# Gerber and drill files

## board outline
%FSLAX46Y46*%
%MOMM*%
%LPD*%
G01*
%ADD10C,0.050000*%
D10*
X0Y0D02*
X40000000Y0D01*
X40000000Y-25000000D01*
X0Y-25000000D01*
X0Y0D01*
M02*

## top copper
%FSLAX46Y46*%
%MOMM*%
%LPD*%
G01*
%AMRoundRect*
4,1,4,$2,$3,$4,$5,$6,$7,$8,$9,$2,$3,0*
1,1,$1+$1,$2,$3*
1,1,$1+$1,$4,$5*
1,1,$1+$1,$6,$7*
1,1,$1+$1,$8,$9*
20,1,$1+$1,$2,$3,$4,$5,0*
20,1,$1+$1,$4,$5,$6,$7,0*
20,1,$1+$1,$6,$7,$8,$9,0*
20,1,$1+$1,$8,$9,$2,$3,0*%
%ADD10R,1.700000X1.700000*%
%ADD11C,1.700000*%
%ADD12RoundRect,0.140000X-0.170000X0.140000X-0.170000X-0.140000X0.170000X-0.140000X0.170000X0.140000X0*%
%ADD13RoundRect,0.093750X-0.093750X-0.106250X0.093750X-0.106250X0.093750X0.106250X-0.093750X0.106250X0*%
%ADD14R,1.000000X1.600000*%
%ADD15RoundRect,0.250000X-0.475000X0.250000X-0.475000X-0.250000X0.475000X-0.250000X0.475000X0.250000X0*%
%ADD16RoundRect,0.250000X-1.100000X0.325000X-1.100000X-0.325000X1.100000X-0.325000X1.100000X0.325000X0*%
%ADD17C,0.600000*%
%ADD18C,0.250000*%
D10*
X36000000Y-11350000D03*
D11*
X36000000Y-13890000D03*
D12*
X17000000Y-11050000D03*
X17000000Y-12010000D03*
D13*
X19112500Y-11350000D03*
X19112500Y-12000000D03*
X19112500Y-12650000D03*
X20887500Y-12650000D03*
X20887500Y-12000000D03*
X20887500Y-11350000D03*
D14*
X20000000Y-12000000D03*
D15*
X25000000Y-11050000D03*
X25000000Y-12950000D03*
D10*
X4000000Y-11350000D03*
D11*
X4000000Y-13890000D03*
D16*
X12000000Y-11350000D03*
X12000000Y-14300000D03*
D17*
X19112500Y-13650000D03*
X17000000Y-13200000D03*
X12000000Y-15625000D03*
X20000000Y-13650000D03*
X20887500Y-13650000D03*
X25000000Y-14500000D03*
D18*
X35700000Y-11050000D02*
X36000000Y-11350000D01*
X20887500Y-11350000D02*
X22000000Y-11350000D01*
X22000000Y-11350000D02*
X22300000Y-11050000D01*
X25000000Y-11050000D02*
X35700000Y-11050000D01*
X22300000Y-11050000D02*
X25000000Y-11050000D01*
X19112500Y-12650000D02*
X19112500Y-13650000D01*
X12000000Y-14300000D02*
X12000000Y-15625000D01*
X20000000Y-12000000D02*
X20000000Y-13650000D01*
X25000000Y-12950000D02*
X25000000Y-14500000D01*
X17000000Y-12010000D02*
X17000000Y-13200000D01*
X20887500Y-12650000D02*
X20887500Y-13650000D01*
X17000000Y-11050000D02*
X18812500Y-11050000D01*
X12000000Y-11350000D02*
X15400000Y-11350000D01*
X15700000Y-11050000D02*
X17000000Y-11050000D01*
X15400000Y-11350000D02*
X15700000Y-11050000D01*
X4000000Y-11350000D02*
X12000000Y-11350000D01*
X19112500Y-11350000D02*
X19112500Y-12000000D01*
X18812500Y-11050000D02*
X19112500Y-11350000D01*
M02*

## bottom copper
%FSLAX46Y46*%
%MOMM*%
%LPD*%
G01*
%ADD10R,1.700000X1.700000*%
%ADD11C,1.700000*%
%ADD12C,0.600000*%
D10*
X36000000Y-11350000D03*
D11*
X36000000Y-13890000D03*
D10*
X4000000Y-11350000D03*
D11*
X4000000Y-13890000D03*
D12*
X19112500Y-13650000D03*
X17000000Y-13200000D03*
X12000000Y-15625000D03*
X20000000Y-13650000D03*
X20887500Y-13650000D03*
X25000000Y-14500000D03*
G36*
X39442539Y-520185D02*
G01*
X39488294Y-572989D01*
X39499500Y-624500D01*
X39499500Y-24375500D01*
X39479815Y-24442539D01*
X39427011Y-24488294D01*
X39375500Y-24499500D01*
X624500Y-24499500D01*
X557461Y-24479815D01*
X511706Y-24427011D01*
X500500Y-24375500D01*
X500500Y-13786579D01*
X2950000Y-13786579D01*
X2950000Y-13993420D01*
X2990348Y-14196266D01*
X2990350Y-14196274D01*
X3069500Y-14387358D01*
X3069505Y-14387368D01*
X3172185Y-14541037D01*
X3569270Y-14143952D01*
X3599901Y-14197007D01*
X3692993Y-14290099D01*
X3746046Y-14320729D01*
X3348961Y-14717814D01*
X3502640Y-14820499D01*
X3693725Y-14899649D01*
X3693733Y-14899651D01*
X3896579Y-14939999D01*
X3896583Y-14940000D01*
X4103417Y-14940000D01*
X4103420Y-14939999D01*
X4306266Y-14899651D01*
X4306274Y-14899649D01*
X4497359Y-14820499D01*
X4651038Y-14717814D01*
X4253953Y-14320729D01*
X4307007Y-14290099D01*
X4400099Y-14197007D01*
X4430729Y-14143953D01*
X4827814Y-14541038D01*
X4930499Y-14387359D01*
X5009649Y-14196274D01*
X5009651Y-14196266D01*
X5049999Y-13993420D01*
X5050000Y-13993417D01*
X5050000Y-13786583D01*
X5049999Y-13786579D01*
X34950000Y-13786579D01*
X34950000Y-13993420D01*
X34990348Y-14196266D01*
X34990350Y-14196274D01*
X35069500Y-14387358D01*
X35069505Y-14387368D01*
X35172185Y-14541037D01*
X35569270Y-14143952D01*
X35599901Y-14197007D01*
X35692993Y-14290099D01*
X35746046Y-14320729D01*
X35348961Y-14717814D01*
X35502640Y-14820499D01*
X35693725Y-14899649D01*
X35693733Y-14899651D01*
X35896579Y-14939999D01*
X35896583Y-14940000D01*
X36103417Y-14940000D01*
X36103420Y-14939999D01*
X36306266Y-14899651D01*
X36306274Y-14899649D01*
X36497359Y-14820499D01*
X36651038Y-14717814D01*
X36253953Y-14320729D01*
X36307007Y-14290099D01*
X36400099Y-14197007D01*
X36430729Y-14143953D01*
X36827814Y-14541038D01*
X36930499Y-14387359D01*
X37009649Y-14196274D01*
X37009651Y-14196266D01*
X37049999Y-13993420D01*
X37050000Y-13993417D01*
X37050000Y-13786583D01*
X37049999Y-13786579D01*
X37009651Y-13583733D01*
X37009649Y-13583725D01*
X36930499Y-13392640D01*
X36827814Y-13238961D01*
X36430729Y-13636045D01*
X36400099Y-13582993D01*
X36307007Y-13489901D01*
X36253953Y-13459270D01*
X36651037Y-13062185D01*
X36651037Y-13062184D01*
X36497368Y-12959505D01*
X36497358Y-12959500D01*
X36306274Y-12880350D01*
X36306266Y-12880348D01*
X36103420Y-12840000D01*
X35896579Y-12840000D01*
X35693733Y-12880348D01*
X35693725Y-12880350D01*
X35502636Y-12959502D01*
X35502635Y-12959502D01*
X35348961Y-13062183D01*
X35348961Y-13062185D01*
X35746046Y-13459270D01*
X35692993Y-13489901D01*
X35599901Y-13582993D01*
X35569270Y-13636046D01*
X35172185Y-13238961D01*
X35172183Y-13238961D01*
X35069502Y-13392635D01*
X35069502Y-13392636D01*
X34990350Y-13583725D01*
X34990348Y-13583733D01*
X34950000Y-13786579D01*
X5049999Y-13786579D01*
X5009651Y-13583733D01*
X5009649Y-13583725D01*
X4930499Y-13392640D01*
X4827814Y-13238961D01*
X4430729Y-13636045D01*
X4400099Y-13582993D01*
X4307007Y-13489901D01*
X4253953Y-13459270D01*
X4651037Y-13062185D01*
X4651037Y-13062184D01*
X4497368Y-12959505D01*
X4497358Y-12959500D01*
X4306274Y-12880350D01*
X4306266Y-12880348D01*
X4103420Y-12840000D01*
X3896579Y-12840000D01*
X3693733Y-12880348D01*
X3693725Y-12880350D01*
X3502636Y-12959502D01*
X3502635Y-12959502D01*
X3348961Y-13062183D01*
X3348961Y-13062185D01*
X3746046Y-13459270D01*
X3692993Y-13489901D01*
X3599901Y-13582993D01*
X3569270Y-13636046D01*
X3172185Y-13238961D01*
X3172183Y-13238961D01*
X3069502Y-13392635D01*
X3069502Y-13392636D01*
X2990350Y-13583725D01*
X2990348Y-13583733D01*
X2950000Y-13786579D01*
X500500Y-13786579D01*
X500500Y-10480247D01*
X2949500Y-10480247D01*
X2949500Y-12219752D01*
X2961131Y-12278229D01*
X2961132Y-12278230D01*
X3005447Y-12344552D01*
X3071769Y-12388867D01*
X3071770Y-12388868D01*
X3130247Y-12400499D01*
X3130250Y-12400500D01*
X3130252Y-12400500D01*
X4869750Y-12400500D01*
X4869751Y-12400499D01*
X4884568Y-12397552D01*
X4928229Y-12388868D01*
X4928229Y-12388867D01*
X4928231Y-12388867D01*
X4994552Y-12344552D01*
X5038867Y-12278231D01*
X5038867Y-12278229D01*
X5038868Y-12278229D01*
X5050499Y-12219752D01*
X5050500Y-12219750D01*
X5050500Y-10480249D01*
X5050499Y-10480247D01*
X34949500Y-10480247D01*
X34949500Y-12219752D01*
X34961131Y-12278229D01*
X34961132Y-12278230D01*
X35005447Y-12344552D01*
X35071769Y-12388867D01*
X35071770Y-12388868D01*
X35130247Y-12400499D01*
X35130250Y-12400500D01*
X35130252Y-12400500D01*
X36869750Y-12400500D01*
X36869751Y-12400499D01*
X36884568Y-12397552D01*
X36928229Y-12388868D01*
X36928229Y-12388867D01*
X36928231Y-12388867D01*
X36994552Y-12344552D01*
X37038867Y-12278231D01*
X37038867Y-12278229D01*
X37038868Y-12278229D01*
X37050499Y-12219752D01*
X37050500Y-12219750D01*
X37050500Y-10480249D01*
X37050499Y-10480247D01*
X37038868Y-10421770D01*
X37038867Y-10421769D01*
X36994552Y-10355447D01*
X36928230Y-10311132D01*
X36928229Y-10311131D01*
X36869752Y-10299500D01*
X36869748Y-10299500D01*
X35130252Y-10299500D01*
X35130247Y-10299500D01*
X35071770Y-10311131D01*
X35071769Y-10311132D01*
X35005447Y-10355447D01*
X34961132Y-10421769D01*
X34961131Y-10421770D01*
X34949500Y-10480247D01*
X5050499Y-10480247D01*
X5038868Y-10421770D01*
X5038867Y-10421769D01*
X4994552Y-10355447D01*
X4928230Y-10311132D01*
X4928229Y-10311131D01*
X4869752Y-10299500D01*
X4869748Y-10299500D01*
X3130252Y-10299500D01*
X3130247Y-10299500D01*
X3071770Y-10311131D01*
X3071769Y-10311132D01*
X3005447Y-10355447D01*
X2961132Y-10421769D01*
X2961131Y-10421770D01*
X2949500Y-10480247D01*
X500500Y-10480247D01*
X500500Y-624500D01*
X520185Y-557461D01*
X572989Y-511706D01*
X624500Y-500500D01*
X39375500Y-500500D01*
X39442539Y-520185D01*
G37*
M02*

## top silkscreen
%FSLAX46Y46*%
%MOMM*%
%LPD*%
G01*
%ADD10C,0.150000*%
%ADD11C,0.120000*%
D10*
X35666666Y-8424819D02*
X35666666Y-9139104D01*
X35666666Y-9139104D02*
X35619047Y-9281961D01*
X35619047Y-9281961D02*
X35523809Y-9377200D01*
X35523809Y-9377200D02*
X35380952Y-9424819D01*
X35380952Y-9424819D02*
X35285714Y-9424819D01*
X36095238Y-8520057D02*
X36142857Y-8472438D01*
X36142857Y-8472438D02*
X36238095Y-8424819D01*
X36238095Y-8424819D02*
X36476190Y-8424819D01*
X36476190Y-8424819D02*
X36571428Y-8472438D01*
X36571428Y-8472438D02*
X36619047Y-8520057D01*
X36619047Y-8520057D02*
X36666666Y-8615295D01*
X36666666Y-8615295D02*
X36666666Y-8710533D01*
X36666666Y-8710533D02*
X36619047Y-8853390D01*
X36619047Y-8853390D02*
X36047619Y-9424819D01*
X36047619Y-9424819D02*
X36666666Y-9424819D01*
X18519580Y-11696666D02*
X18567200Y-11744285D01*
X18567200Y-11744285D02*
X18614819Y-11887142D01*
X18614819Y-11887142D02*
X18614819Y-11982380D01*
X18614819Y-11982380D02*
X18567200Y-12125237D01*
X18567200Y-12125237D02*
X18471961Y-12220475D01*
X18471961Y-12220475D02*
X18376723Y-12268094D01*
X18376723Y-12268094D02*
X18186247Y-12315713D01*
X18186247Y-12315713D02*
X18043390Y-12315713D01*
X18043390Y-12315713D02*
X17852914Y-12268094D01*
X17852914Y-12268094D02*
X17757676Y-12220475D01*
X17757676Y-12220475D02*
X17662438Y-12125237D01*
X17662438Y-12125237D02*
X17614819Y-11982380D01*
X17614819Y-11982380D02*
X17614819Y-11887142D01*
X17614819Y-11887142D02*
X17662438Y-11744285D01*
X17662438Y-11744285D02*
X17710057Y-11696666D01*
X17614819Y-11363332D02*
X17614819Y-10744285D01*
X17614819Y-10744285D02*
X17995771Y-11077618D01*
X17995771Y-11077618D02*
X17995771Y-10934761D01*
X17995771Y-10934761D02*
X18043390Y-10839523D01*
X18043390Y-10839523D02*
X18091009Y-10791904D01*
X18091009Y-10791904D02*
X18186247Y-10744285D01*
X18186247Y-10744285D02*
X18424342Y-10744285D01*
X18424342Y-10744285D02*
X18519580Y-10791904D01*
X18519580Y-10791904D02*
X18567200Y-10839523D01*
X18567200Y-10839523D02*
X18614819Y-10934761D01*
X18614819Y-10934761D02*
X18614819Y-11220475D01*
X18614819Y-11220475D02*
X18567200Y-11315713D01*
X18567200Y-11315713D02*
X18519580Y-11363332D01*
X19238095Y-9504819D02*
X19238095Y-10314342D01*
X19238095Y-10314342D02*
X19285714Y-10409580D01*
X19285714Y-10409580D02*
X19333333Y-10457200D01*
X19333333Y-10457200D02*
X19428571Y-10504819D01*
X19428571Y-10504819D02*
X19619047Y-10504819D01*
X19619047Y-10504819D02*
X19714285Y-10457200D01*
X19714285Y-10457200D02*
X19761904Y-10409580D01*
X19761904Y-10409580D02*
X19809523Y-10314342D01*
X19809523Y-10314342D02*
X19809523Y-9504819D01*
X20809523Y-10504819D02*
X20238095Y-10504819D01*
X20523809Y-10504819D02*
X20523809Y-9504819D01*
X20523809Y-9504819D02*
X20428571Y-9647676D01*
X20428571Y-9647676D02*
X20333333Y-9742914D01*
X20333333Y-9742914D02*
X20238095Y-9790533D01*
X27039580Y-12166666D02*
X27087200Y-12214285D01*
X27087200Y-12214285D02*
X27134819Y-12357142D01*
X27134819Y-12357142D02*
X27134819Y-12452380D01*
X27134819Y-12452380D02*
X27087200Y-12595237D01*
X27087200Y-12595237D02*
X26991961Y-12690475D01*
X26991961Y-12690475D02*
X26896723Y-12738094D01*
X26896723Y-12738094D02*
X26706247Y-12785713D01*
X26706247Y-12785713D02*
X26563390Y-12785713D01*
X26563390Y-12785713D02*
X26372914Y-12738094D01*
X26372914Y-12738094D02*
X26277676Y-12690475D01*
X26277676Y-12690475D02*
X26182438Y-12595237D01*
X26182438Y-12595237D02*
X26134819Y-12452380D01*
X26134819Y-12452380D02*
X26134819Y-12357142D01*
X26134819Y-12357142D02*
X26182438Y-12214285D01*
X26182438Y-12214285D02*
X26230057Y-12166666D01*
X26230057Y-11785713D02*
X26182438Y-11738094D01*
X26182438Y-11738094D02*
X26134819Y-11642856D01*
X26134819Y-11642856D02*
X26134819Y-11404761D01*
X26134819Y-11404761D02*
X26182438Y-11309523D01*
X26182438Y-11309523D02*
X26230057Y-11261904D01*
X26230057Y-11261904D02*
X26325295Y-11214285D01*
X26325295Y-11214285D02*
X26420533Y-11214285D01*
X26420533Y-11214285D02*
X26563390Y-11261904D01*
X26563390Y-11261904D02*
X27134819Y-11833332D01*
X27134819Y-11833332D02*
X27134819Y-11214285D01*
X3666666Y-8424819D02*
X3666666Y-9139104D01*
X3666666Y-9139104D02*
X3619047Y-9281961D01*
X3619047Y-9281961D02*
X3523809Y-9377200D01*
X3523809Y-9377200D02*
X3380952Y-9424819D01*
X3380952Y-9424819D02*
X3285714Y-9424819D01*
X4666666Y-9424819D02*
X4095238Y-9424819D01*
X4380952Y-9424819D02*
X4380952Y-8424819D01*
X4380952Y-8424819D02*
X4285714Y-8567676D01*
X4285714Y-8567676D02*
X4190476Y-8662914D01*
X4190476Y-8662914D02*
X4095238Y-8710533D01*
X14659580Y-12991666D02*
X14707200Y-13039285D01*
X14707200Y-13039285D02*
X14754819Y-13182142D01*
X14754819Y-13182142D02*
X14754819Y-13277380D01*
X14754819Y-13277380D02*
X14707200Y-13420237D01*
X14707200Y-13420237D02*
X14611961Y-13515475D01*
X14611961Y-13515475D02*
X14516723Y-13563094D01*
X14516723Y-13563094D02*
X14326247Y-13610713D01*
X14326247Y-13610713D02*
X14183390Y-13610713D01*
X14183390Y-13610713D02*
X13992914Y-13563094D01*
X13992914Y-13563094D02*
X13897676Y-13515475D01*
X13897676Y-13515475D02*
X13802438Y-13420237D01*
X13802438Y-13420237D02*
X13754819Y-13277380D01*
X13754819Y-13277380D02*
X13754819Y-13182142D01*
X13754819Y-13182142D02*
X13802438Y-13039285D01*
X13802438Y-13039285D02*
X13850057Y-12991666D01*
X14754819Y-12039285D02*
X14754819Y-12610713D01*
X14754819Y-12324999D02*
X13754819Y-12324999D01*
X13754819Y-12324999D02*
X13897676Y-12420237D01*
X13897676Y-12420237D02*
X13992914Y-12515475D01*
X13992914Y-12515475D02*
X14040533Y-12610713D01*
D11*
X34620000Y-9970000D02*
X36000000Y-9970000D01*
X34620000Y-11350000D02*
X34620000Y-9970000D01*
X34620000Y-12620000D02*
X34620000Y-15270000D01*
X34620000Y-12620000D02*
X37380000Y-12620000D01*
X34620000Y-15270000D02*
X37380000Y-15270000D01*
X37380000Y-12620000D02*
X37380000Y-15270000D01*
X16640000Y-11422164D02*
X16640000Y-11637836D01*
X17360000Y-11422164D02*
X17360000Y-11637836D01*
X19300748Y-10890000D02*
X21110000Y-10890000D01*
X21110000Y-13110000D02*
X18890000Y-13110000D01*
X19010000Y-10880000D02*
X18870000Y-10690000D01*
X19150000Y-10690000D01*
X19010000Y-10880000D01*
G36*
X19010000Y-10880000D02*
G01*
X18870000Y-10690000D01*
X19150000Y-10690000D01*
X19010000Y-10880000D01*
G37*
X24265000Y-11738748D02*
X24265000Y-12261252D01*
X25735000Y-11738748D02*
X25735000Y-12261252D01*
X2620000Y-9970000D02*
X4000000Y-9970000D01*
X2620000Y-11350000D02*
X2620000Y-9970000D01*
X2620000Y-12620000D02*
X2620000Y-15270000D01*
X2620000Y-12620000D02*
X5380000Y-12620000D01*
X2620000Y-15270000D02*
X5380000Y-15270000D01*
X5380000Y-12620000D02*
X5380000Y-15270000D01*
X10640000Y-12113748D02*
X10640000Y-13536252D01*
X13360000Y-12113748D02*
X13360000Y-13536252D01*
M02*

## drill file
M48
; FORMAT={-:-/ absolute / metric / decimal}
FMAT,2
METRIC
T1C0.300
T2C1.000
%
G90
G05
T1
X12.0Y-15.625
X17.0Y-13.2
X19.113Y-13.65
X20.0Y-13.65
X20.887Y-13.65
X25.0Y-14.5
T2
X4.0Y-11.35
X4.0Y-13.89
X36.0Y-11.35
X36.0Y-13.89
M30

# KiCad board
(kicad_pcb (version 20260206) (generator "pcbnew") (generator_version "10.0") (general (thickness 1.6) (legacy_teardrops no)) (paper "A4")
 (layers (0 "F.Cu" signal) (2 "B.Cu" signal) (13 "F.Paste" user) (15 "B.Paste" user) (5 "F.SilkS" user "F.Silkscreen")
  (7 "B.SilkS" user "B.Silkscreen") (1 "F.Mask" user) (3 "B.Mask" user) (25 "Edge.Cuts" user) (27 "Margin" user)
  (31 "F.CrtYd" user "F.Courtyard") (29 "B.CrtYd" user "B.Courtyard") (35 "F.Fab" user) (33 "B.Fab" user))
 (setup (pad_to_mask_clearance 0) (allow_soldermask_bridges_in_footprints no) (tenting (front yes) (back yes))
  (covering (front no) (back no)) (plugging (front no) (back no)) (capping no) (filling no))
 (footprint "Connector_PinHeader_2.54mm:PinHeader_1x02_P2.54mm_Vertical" (layer "F.Cu") (at 36 11.35)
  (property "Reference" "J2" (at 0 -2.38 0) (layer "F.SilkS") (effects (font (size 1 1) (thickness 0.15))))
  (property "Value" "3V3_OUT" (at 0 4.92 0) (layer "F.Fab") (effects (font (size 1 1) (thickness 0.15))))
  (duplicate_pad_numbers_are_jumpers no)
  (fp_line (start -1.38 -1.38) (end 0 -1.38) (stroke (width 0.12) (type solid)) (layer "F.SilkS"))
  (fp_line (start -1.38 0) (end -1.38 -1.38) (stroke (width 0.12) (type solid)) (layer "F.SilkS"))
  (fp_line (start -1.38 1.27) (end -1.38 3.92) (stroke (width 0.12) (type solid)) (layer "F.SilkS"))
  (fp_line (start -1.38 1.27) (end 1.38 1.27) (stroke (width 0.12) (type solid)) (layer "F.SilkS"))
  (fp_line (start -1.38 3.92) (end 1.38 3.92) (stroke (width 0.12) (type solid)) (layer "F.SilkS"))
  (fp_line (start 1.38 1.27) (end 1.38 3.92) (stroke (width 0.12) (type solid)) (layer "F.SilkS"))
  (pad "1" thru_hole rect (at 0 0) (size 1.7 1.7) (drill 1) (layers "*.Cu" "*.Mask") (remove_unused_layers no) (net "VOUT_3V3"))
  (pad "2" thru_hole circle (at 0 2.54) (size 1.7 1.7) (drill 1) (layers "*.Cu" "*.Mask") (remove_unused_layers no) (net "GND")))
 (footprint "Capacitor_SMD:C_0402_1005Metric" (layer "F.Cu") (at 17 11.53 -90)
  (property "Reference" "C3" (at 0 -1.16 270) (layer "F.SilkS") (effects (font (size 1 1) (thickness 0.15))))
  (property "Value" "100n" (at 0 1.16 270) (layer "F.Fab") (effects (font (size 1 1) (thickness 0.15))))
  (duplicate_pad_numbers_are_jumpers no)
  (fp_line (start -0.107836 0.36) (end 0.107836 0.36) (stroke (width 0.12) (type solid)) (layer "F.SilkS"))
  (fp_line (start -0.107836 -0.36) (end 0.107836 -0.36) (stroke (width 0.12) (type solid)) (layer "F.SilkS"))
  (pad "1" smd roundrect (at -0.48 0 270) (size 0.56 0.62) (layers "F.Cu" "F.Mask" "F.Paste") (roundrect_rratio 0.25) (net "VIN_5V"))
  (pad "2" smd roundrect (at 0.48 0 270) (size 0.56 0.62) (layers "F.Cu" "F.Mask" "F.Paste") (roundrect_rratio 0.25) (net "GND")))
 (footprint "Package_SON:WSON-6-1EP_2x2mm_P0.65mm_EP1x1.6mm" (layer "F.Cu") (at 20 12)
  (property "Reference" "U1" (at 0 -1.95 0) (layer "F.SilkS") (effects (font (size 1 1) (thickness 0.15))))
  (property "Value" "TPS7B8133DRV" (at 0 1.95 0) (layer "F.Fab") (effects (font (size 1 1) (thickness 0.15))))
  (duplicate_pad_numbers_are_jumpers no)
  (fp_line (start -0.699252 -1.11) (end 1.11 -1.11) (stroke (width 0.12) (type solid)) (layer "F.SilkS"))
  (fp_line (start 1.11 1.11) (end -1.11 1.11) (stroke (width 0.12) (type solid)) (layer "F.SilkS"))
  (fp_poly (pts (xy -0.99 -1.12) (xy -1.13 -1.31) (xy -0.85 -1.31)) (stroke (width 0.12) (type solid)) (fill yes) (layer "F.SilkS"))
  (pad "" smd roundrect (at 0 -0.4) (size 0.81 0.64) (layers "F.Paste") (roundrect_rratio 0.25))
  (pad "" smd roundrect (at 0 0.4) (size 0.81 0.64) (layers "F.Paste") (roundrect_rratio 0.25))
  (pad "1" smd roundrect (at -0.8875 -0.65) (size 0.375 0.4) (layers "F.Cu" "F.Mask" "F.Paste") (roundrect_rratio 0.25) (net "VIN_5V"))
  (pad "2" smd roundrect (at -0.8875 0) (size 0.375 0.4) (layers "F.Cu" "F.Mask" "F.Paste") (roundrect_rratio 0.25) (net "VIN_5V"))
  (pad "3" smd roundrect (at -0.8875 0.65) (size 0.375 0.4) (layers "F.Cu" "F.Mask" "F.Paste") (roundrect_rratio 0.25) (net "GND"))
  (pad "4" smd roundrect (at 0.8875 0.65) (size 0.375 0.4) (layers "F.Cu" "F.Mask" "F.Paste") (roundrect_rratio 0.25) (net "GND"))
  (pad "5" smd roundrect (at 0.8875 0) (size 0.375 0.4) (layers "F.Cu" "F.Mask" "F.Paste") (roundrect_rratio 0.25)
   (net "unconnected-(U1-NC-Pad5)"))
  (pad "6" smd roundrect (at 0.8875 -0.65) (size 0.375 0.4) (layers "F.Cu" "F.Mask" "F.Paste") (roundrect_rratio 0.25) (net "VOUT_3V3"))
  (pad "7" smd rect (at 0 0) (size 1 1.6) (layers "F.Cu" "F.Mask") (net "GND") (zone_connect 2)))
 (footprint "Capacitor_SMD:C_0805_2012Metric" (layer "F.Cu") (at 25 12 -90)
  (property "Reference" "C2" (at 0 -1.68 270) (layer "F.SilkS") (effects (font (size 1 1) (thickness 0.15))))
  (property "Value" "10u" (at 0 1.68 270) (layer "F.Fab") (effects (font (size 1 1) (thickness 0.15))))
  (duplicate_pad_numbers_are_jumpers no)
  (fp_line (start -0.261252 0.735) (end 0.261252 0.735) (stroke (width 0.12) (type solid)) (layer "F.SilkS"))
  (fp_line (start -0.261252 -0.735) (end 0.261252 -0.735) (stroke (width 0.12) (type solid)) (layer "F.SilkS"))
  (pad "1" smd roundrect (at -0.95 0 270) (size 1 1.45) (layers "F.Cu" "F.Mask" "F.Paste") (roundrect_rratio 0.25) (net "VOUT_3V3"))
  (pad "2" smd roundrect (at 0.95 0 270) (size 1 1.45) (layers "F.Cu" "F.Mask" "F.Paste") (roundrect_rratio 0.25) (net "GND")))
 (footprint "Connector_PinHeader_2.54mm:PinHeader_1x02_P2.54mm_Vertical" (layer "F.Cu") (at 4 11.35)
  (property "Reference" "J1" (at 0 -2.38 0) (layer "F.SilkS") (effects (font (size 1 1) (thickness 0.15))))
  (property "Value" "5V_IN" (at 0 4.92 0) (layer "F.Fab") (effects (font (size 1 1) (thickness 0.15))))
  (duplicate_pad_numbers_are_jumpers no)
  (fp_line (start -1.38 -1.38) (end 0 -1.38) (stroke (width 0.12) (type solid)) (layer "F.SilkS"))
  (fp_line (start -1.38 0) (end -1.38 -1.38) (stroke (width 0.12) (type solid)) (layer "F.SilkS"))
  (fp_line (start -1.38 1.27) (end -1.38 3.92) (stroke (width 0.12) (type solid)) (layer "F.SilkS"))
  (fp_line (start -1.38 1.27) (end 1.38 1.27) (stroke (width 0.12) (type solid)) (layer "F.SilkS"))
  (fp_line (start -1.38 3.92) (end 1.38 3.92) (stroke (width 0.12) (type solid)) (layer "F.SilkS"))
  (fp_line (start 1.38 1.27) (end 1.38 3.92) (stroke (width 0.12) (type solid)) (layer "F.SilkS"))
  (pad "1" thru_hole rect (at 0 0) (size 1.7 1.7) (drill 1) (layers "*.Cu" "*.Mask") (remove_unused_layers no) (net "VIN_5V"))
  (pad "2" thru_hole circle (at 0 2.54) (size 1.7 1.7) (drill 1) (layers "*.Cu" "*.Mask") (remove_unused_layers no) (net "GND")))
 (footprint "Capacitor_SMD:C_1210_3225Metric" (layer "F.Cu") (at 12 12.825 -90)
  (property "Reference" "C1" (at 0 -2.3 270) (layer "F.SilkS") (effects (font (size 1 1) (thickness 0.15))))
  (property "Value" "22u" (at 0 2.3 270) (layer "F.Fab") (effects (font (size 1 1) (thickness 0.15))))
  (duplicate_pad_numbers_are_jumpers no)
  (fp_line (start -0.711252 1.36) (end 0.711252 1.36) (stroke (width 0.12) (type solid)) (layer "F.SilkS"))
  (fp_line (start -0.711252 -1.36) (end 0.711252 -1.36) (stroke (width 0.12) (type solid)) (layer "F.SilkS"))
  (pad "1" smd roundrect (at -1.475 0 270) (size 1.15 2.7) (layers "F.Cu" "F.Mask" "F.Paste") (roundrect_rratio 0.217391) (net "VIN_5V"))
  (pad "2" smd roundrect (at 1.475 0 270) (size 1.15 2.7) (layers "F.Cu" "F.Mask" "F.Paste") (roundrect_rratio 0.217391) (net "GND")))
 (gr_rect (start 0 0) (end 40 25) (stroke (width 0.05) (type default)) (fill no) (layer "Edge.Cuts"))
 (segment (start 35.7 11.05) (end 36 11.35) (width 0.25) (layer "F.Cu") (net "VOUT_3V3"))
 (segment (start 20.8875 11.35) (end 22 11.35) (width 0.25) (layer "F.Cu") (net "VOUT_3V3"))
 (segment (start 22 11.35) (end 22.3 11.05) (width 0.25) (layer "F.Cu") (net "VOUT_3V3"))
 (segment (start 25 11.05) (end 35.7 11.05) (width 0.25) (layer "F.Cu") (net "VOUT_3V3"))
 (segment (start 22.3 11.05) (end 25 11.05) (width 0.25) (layer "F.Cu") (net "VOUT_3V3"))
 (segment (start 19.1125 12.65) (end 19.1125 13.65) (width 0.25) (layer "F.Cu") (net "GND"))
 (segment (start 12 14.3) (end 12 15.625) (width 0.25) (layer "F.Cu") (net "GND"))
 (segment (start 20 12) (end 20 13.65) (width 0.25) (layer "F.Cu") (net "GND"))
 (segment (start 25 12.95) (end 25 14.5) (width 0.25) (layer "F.Cu") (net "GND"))
 (segment (start 17 12.01) (end 17 13.2) (width 0.25) (layer "F.Cu") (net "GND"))
 (segment (start 20.8875 12.65) (end 20.8875 13.65) (width 0.25) (layer "F.Cu") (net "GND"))
 (via (at 19.1125 13.65) (size 0.6) (drill 0.3) (layers "F.Cu" "B.Cu") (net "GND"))
 (via (at 17 13.2) (size 0.6) (drill 0.3) (layers "F.Cu" "B.Cu") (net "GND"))
 (via (at 12 15.625) (size 0.6) (drill 0.3) (layers "F.Cu" "B.Cu") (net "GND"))
 (via (at 20 13.65) (size 0.6) (drill 0.3) (layers "F.Cu" "B.Cu") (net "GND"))
 (via (at 20.8875 13.65) (size 0.6) (drill 0.3) (layers "F.Cu" "B.Cu") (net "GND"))
 (via (at 25 14.5) (size 0.6) (drill 0.3) (layers "F.Cu" "B.Cu") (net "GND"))
 (segment (start 17 11.05) (end 18.8125 11.05) (width 0.25) (layer "F.Cu") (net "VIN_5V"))
 (segment (start 12 11.35) (end 15.4 11.35) (width 0.25) (layer "F.Cu") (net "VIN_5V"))
 (segment (start 15.7 11.05) (end 17 11.05) (width 0.25) (layer "F.Cu") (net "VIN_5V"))
 (segment (start 15.4 11.35) (end 15.7 11.05) (width 0.25) (layer "F.Cu") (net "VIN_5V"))
 (segment (start 4 11.35) (end 12 11.35) (width 0.25) (layer "F.Cu") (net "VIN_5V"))
 (segment (start 19.1125 11.35) (end 19.1125 12) (width 0.25) (layer "F.Cu") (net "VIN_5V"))
 (segment (start 18.8125 11.05) (end 19.1125 11.35) (width 0.25) (layer "F.Cu") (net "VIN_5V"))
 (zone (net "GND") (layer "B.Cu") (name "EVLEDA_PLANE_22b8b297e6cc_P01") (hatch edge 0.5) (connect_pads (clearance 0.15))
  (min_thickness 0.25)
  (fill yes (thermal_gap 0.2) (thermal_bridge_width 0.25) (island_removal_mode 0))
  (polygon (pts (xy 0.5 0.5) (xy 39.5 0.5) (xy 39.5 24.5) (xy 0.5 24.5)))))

